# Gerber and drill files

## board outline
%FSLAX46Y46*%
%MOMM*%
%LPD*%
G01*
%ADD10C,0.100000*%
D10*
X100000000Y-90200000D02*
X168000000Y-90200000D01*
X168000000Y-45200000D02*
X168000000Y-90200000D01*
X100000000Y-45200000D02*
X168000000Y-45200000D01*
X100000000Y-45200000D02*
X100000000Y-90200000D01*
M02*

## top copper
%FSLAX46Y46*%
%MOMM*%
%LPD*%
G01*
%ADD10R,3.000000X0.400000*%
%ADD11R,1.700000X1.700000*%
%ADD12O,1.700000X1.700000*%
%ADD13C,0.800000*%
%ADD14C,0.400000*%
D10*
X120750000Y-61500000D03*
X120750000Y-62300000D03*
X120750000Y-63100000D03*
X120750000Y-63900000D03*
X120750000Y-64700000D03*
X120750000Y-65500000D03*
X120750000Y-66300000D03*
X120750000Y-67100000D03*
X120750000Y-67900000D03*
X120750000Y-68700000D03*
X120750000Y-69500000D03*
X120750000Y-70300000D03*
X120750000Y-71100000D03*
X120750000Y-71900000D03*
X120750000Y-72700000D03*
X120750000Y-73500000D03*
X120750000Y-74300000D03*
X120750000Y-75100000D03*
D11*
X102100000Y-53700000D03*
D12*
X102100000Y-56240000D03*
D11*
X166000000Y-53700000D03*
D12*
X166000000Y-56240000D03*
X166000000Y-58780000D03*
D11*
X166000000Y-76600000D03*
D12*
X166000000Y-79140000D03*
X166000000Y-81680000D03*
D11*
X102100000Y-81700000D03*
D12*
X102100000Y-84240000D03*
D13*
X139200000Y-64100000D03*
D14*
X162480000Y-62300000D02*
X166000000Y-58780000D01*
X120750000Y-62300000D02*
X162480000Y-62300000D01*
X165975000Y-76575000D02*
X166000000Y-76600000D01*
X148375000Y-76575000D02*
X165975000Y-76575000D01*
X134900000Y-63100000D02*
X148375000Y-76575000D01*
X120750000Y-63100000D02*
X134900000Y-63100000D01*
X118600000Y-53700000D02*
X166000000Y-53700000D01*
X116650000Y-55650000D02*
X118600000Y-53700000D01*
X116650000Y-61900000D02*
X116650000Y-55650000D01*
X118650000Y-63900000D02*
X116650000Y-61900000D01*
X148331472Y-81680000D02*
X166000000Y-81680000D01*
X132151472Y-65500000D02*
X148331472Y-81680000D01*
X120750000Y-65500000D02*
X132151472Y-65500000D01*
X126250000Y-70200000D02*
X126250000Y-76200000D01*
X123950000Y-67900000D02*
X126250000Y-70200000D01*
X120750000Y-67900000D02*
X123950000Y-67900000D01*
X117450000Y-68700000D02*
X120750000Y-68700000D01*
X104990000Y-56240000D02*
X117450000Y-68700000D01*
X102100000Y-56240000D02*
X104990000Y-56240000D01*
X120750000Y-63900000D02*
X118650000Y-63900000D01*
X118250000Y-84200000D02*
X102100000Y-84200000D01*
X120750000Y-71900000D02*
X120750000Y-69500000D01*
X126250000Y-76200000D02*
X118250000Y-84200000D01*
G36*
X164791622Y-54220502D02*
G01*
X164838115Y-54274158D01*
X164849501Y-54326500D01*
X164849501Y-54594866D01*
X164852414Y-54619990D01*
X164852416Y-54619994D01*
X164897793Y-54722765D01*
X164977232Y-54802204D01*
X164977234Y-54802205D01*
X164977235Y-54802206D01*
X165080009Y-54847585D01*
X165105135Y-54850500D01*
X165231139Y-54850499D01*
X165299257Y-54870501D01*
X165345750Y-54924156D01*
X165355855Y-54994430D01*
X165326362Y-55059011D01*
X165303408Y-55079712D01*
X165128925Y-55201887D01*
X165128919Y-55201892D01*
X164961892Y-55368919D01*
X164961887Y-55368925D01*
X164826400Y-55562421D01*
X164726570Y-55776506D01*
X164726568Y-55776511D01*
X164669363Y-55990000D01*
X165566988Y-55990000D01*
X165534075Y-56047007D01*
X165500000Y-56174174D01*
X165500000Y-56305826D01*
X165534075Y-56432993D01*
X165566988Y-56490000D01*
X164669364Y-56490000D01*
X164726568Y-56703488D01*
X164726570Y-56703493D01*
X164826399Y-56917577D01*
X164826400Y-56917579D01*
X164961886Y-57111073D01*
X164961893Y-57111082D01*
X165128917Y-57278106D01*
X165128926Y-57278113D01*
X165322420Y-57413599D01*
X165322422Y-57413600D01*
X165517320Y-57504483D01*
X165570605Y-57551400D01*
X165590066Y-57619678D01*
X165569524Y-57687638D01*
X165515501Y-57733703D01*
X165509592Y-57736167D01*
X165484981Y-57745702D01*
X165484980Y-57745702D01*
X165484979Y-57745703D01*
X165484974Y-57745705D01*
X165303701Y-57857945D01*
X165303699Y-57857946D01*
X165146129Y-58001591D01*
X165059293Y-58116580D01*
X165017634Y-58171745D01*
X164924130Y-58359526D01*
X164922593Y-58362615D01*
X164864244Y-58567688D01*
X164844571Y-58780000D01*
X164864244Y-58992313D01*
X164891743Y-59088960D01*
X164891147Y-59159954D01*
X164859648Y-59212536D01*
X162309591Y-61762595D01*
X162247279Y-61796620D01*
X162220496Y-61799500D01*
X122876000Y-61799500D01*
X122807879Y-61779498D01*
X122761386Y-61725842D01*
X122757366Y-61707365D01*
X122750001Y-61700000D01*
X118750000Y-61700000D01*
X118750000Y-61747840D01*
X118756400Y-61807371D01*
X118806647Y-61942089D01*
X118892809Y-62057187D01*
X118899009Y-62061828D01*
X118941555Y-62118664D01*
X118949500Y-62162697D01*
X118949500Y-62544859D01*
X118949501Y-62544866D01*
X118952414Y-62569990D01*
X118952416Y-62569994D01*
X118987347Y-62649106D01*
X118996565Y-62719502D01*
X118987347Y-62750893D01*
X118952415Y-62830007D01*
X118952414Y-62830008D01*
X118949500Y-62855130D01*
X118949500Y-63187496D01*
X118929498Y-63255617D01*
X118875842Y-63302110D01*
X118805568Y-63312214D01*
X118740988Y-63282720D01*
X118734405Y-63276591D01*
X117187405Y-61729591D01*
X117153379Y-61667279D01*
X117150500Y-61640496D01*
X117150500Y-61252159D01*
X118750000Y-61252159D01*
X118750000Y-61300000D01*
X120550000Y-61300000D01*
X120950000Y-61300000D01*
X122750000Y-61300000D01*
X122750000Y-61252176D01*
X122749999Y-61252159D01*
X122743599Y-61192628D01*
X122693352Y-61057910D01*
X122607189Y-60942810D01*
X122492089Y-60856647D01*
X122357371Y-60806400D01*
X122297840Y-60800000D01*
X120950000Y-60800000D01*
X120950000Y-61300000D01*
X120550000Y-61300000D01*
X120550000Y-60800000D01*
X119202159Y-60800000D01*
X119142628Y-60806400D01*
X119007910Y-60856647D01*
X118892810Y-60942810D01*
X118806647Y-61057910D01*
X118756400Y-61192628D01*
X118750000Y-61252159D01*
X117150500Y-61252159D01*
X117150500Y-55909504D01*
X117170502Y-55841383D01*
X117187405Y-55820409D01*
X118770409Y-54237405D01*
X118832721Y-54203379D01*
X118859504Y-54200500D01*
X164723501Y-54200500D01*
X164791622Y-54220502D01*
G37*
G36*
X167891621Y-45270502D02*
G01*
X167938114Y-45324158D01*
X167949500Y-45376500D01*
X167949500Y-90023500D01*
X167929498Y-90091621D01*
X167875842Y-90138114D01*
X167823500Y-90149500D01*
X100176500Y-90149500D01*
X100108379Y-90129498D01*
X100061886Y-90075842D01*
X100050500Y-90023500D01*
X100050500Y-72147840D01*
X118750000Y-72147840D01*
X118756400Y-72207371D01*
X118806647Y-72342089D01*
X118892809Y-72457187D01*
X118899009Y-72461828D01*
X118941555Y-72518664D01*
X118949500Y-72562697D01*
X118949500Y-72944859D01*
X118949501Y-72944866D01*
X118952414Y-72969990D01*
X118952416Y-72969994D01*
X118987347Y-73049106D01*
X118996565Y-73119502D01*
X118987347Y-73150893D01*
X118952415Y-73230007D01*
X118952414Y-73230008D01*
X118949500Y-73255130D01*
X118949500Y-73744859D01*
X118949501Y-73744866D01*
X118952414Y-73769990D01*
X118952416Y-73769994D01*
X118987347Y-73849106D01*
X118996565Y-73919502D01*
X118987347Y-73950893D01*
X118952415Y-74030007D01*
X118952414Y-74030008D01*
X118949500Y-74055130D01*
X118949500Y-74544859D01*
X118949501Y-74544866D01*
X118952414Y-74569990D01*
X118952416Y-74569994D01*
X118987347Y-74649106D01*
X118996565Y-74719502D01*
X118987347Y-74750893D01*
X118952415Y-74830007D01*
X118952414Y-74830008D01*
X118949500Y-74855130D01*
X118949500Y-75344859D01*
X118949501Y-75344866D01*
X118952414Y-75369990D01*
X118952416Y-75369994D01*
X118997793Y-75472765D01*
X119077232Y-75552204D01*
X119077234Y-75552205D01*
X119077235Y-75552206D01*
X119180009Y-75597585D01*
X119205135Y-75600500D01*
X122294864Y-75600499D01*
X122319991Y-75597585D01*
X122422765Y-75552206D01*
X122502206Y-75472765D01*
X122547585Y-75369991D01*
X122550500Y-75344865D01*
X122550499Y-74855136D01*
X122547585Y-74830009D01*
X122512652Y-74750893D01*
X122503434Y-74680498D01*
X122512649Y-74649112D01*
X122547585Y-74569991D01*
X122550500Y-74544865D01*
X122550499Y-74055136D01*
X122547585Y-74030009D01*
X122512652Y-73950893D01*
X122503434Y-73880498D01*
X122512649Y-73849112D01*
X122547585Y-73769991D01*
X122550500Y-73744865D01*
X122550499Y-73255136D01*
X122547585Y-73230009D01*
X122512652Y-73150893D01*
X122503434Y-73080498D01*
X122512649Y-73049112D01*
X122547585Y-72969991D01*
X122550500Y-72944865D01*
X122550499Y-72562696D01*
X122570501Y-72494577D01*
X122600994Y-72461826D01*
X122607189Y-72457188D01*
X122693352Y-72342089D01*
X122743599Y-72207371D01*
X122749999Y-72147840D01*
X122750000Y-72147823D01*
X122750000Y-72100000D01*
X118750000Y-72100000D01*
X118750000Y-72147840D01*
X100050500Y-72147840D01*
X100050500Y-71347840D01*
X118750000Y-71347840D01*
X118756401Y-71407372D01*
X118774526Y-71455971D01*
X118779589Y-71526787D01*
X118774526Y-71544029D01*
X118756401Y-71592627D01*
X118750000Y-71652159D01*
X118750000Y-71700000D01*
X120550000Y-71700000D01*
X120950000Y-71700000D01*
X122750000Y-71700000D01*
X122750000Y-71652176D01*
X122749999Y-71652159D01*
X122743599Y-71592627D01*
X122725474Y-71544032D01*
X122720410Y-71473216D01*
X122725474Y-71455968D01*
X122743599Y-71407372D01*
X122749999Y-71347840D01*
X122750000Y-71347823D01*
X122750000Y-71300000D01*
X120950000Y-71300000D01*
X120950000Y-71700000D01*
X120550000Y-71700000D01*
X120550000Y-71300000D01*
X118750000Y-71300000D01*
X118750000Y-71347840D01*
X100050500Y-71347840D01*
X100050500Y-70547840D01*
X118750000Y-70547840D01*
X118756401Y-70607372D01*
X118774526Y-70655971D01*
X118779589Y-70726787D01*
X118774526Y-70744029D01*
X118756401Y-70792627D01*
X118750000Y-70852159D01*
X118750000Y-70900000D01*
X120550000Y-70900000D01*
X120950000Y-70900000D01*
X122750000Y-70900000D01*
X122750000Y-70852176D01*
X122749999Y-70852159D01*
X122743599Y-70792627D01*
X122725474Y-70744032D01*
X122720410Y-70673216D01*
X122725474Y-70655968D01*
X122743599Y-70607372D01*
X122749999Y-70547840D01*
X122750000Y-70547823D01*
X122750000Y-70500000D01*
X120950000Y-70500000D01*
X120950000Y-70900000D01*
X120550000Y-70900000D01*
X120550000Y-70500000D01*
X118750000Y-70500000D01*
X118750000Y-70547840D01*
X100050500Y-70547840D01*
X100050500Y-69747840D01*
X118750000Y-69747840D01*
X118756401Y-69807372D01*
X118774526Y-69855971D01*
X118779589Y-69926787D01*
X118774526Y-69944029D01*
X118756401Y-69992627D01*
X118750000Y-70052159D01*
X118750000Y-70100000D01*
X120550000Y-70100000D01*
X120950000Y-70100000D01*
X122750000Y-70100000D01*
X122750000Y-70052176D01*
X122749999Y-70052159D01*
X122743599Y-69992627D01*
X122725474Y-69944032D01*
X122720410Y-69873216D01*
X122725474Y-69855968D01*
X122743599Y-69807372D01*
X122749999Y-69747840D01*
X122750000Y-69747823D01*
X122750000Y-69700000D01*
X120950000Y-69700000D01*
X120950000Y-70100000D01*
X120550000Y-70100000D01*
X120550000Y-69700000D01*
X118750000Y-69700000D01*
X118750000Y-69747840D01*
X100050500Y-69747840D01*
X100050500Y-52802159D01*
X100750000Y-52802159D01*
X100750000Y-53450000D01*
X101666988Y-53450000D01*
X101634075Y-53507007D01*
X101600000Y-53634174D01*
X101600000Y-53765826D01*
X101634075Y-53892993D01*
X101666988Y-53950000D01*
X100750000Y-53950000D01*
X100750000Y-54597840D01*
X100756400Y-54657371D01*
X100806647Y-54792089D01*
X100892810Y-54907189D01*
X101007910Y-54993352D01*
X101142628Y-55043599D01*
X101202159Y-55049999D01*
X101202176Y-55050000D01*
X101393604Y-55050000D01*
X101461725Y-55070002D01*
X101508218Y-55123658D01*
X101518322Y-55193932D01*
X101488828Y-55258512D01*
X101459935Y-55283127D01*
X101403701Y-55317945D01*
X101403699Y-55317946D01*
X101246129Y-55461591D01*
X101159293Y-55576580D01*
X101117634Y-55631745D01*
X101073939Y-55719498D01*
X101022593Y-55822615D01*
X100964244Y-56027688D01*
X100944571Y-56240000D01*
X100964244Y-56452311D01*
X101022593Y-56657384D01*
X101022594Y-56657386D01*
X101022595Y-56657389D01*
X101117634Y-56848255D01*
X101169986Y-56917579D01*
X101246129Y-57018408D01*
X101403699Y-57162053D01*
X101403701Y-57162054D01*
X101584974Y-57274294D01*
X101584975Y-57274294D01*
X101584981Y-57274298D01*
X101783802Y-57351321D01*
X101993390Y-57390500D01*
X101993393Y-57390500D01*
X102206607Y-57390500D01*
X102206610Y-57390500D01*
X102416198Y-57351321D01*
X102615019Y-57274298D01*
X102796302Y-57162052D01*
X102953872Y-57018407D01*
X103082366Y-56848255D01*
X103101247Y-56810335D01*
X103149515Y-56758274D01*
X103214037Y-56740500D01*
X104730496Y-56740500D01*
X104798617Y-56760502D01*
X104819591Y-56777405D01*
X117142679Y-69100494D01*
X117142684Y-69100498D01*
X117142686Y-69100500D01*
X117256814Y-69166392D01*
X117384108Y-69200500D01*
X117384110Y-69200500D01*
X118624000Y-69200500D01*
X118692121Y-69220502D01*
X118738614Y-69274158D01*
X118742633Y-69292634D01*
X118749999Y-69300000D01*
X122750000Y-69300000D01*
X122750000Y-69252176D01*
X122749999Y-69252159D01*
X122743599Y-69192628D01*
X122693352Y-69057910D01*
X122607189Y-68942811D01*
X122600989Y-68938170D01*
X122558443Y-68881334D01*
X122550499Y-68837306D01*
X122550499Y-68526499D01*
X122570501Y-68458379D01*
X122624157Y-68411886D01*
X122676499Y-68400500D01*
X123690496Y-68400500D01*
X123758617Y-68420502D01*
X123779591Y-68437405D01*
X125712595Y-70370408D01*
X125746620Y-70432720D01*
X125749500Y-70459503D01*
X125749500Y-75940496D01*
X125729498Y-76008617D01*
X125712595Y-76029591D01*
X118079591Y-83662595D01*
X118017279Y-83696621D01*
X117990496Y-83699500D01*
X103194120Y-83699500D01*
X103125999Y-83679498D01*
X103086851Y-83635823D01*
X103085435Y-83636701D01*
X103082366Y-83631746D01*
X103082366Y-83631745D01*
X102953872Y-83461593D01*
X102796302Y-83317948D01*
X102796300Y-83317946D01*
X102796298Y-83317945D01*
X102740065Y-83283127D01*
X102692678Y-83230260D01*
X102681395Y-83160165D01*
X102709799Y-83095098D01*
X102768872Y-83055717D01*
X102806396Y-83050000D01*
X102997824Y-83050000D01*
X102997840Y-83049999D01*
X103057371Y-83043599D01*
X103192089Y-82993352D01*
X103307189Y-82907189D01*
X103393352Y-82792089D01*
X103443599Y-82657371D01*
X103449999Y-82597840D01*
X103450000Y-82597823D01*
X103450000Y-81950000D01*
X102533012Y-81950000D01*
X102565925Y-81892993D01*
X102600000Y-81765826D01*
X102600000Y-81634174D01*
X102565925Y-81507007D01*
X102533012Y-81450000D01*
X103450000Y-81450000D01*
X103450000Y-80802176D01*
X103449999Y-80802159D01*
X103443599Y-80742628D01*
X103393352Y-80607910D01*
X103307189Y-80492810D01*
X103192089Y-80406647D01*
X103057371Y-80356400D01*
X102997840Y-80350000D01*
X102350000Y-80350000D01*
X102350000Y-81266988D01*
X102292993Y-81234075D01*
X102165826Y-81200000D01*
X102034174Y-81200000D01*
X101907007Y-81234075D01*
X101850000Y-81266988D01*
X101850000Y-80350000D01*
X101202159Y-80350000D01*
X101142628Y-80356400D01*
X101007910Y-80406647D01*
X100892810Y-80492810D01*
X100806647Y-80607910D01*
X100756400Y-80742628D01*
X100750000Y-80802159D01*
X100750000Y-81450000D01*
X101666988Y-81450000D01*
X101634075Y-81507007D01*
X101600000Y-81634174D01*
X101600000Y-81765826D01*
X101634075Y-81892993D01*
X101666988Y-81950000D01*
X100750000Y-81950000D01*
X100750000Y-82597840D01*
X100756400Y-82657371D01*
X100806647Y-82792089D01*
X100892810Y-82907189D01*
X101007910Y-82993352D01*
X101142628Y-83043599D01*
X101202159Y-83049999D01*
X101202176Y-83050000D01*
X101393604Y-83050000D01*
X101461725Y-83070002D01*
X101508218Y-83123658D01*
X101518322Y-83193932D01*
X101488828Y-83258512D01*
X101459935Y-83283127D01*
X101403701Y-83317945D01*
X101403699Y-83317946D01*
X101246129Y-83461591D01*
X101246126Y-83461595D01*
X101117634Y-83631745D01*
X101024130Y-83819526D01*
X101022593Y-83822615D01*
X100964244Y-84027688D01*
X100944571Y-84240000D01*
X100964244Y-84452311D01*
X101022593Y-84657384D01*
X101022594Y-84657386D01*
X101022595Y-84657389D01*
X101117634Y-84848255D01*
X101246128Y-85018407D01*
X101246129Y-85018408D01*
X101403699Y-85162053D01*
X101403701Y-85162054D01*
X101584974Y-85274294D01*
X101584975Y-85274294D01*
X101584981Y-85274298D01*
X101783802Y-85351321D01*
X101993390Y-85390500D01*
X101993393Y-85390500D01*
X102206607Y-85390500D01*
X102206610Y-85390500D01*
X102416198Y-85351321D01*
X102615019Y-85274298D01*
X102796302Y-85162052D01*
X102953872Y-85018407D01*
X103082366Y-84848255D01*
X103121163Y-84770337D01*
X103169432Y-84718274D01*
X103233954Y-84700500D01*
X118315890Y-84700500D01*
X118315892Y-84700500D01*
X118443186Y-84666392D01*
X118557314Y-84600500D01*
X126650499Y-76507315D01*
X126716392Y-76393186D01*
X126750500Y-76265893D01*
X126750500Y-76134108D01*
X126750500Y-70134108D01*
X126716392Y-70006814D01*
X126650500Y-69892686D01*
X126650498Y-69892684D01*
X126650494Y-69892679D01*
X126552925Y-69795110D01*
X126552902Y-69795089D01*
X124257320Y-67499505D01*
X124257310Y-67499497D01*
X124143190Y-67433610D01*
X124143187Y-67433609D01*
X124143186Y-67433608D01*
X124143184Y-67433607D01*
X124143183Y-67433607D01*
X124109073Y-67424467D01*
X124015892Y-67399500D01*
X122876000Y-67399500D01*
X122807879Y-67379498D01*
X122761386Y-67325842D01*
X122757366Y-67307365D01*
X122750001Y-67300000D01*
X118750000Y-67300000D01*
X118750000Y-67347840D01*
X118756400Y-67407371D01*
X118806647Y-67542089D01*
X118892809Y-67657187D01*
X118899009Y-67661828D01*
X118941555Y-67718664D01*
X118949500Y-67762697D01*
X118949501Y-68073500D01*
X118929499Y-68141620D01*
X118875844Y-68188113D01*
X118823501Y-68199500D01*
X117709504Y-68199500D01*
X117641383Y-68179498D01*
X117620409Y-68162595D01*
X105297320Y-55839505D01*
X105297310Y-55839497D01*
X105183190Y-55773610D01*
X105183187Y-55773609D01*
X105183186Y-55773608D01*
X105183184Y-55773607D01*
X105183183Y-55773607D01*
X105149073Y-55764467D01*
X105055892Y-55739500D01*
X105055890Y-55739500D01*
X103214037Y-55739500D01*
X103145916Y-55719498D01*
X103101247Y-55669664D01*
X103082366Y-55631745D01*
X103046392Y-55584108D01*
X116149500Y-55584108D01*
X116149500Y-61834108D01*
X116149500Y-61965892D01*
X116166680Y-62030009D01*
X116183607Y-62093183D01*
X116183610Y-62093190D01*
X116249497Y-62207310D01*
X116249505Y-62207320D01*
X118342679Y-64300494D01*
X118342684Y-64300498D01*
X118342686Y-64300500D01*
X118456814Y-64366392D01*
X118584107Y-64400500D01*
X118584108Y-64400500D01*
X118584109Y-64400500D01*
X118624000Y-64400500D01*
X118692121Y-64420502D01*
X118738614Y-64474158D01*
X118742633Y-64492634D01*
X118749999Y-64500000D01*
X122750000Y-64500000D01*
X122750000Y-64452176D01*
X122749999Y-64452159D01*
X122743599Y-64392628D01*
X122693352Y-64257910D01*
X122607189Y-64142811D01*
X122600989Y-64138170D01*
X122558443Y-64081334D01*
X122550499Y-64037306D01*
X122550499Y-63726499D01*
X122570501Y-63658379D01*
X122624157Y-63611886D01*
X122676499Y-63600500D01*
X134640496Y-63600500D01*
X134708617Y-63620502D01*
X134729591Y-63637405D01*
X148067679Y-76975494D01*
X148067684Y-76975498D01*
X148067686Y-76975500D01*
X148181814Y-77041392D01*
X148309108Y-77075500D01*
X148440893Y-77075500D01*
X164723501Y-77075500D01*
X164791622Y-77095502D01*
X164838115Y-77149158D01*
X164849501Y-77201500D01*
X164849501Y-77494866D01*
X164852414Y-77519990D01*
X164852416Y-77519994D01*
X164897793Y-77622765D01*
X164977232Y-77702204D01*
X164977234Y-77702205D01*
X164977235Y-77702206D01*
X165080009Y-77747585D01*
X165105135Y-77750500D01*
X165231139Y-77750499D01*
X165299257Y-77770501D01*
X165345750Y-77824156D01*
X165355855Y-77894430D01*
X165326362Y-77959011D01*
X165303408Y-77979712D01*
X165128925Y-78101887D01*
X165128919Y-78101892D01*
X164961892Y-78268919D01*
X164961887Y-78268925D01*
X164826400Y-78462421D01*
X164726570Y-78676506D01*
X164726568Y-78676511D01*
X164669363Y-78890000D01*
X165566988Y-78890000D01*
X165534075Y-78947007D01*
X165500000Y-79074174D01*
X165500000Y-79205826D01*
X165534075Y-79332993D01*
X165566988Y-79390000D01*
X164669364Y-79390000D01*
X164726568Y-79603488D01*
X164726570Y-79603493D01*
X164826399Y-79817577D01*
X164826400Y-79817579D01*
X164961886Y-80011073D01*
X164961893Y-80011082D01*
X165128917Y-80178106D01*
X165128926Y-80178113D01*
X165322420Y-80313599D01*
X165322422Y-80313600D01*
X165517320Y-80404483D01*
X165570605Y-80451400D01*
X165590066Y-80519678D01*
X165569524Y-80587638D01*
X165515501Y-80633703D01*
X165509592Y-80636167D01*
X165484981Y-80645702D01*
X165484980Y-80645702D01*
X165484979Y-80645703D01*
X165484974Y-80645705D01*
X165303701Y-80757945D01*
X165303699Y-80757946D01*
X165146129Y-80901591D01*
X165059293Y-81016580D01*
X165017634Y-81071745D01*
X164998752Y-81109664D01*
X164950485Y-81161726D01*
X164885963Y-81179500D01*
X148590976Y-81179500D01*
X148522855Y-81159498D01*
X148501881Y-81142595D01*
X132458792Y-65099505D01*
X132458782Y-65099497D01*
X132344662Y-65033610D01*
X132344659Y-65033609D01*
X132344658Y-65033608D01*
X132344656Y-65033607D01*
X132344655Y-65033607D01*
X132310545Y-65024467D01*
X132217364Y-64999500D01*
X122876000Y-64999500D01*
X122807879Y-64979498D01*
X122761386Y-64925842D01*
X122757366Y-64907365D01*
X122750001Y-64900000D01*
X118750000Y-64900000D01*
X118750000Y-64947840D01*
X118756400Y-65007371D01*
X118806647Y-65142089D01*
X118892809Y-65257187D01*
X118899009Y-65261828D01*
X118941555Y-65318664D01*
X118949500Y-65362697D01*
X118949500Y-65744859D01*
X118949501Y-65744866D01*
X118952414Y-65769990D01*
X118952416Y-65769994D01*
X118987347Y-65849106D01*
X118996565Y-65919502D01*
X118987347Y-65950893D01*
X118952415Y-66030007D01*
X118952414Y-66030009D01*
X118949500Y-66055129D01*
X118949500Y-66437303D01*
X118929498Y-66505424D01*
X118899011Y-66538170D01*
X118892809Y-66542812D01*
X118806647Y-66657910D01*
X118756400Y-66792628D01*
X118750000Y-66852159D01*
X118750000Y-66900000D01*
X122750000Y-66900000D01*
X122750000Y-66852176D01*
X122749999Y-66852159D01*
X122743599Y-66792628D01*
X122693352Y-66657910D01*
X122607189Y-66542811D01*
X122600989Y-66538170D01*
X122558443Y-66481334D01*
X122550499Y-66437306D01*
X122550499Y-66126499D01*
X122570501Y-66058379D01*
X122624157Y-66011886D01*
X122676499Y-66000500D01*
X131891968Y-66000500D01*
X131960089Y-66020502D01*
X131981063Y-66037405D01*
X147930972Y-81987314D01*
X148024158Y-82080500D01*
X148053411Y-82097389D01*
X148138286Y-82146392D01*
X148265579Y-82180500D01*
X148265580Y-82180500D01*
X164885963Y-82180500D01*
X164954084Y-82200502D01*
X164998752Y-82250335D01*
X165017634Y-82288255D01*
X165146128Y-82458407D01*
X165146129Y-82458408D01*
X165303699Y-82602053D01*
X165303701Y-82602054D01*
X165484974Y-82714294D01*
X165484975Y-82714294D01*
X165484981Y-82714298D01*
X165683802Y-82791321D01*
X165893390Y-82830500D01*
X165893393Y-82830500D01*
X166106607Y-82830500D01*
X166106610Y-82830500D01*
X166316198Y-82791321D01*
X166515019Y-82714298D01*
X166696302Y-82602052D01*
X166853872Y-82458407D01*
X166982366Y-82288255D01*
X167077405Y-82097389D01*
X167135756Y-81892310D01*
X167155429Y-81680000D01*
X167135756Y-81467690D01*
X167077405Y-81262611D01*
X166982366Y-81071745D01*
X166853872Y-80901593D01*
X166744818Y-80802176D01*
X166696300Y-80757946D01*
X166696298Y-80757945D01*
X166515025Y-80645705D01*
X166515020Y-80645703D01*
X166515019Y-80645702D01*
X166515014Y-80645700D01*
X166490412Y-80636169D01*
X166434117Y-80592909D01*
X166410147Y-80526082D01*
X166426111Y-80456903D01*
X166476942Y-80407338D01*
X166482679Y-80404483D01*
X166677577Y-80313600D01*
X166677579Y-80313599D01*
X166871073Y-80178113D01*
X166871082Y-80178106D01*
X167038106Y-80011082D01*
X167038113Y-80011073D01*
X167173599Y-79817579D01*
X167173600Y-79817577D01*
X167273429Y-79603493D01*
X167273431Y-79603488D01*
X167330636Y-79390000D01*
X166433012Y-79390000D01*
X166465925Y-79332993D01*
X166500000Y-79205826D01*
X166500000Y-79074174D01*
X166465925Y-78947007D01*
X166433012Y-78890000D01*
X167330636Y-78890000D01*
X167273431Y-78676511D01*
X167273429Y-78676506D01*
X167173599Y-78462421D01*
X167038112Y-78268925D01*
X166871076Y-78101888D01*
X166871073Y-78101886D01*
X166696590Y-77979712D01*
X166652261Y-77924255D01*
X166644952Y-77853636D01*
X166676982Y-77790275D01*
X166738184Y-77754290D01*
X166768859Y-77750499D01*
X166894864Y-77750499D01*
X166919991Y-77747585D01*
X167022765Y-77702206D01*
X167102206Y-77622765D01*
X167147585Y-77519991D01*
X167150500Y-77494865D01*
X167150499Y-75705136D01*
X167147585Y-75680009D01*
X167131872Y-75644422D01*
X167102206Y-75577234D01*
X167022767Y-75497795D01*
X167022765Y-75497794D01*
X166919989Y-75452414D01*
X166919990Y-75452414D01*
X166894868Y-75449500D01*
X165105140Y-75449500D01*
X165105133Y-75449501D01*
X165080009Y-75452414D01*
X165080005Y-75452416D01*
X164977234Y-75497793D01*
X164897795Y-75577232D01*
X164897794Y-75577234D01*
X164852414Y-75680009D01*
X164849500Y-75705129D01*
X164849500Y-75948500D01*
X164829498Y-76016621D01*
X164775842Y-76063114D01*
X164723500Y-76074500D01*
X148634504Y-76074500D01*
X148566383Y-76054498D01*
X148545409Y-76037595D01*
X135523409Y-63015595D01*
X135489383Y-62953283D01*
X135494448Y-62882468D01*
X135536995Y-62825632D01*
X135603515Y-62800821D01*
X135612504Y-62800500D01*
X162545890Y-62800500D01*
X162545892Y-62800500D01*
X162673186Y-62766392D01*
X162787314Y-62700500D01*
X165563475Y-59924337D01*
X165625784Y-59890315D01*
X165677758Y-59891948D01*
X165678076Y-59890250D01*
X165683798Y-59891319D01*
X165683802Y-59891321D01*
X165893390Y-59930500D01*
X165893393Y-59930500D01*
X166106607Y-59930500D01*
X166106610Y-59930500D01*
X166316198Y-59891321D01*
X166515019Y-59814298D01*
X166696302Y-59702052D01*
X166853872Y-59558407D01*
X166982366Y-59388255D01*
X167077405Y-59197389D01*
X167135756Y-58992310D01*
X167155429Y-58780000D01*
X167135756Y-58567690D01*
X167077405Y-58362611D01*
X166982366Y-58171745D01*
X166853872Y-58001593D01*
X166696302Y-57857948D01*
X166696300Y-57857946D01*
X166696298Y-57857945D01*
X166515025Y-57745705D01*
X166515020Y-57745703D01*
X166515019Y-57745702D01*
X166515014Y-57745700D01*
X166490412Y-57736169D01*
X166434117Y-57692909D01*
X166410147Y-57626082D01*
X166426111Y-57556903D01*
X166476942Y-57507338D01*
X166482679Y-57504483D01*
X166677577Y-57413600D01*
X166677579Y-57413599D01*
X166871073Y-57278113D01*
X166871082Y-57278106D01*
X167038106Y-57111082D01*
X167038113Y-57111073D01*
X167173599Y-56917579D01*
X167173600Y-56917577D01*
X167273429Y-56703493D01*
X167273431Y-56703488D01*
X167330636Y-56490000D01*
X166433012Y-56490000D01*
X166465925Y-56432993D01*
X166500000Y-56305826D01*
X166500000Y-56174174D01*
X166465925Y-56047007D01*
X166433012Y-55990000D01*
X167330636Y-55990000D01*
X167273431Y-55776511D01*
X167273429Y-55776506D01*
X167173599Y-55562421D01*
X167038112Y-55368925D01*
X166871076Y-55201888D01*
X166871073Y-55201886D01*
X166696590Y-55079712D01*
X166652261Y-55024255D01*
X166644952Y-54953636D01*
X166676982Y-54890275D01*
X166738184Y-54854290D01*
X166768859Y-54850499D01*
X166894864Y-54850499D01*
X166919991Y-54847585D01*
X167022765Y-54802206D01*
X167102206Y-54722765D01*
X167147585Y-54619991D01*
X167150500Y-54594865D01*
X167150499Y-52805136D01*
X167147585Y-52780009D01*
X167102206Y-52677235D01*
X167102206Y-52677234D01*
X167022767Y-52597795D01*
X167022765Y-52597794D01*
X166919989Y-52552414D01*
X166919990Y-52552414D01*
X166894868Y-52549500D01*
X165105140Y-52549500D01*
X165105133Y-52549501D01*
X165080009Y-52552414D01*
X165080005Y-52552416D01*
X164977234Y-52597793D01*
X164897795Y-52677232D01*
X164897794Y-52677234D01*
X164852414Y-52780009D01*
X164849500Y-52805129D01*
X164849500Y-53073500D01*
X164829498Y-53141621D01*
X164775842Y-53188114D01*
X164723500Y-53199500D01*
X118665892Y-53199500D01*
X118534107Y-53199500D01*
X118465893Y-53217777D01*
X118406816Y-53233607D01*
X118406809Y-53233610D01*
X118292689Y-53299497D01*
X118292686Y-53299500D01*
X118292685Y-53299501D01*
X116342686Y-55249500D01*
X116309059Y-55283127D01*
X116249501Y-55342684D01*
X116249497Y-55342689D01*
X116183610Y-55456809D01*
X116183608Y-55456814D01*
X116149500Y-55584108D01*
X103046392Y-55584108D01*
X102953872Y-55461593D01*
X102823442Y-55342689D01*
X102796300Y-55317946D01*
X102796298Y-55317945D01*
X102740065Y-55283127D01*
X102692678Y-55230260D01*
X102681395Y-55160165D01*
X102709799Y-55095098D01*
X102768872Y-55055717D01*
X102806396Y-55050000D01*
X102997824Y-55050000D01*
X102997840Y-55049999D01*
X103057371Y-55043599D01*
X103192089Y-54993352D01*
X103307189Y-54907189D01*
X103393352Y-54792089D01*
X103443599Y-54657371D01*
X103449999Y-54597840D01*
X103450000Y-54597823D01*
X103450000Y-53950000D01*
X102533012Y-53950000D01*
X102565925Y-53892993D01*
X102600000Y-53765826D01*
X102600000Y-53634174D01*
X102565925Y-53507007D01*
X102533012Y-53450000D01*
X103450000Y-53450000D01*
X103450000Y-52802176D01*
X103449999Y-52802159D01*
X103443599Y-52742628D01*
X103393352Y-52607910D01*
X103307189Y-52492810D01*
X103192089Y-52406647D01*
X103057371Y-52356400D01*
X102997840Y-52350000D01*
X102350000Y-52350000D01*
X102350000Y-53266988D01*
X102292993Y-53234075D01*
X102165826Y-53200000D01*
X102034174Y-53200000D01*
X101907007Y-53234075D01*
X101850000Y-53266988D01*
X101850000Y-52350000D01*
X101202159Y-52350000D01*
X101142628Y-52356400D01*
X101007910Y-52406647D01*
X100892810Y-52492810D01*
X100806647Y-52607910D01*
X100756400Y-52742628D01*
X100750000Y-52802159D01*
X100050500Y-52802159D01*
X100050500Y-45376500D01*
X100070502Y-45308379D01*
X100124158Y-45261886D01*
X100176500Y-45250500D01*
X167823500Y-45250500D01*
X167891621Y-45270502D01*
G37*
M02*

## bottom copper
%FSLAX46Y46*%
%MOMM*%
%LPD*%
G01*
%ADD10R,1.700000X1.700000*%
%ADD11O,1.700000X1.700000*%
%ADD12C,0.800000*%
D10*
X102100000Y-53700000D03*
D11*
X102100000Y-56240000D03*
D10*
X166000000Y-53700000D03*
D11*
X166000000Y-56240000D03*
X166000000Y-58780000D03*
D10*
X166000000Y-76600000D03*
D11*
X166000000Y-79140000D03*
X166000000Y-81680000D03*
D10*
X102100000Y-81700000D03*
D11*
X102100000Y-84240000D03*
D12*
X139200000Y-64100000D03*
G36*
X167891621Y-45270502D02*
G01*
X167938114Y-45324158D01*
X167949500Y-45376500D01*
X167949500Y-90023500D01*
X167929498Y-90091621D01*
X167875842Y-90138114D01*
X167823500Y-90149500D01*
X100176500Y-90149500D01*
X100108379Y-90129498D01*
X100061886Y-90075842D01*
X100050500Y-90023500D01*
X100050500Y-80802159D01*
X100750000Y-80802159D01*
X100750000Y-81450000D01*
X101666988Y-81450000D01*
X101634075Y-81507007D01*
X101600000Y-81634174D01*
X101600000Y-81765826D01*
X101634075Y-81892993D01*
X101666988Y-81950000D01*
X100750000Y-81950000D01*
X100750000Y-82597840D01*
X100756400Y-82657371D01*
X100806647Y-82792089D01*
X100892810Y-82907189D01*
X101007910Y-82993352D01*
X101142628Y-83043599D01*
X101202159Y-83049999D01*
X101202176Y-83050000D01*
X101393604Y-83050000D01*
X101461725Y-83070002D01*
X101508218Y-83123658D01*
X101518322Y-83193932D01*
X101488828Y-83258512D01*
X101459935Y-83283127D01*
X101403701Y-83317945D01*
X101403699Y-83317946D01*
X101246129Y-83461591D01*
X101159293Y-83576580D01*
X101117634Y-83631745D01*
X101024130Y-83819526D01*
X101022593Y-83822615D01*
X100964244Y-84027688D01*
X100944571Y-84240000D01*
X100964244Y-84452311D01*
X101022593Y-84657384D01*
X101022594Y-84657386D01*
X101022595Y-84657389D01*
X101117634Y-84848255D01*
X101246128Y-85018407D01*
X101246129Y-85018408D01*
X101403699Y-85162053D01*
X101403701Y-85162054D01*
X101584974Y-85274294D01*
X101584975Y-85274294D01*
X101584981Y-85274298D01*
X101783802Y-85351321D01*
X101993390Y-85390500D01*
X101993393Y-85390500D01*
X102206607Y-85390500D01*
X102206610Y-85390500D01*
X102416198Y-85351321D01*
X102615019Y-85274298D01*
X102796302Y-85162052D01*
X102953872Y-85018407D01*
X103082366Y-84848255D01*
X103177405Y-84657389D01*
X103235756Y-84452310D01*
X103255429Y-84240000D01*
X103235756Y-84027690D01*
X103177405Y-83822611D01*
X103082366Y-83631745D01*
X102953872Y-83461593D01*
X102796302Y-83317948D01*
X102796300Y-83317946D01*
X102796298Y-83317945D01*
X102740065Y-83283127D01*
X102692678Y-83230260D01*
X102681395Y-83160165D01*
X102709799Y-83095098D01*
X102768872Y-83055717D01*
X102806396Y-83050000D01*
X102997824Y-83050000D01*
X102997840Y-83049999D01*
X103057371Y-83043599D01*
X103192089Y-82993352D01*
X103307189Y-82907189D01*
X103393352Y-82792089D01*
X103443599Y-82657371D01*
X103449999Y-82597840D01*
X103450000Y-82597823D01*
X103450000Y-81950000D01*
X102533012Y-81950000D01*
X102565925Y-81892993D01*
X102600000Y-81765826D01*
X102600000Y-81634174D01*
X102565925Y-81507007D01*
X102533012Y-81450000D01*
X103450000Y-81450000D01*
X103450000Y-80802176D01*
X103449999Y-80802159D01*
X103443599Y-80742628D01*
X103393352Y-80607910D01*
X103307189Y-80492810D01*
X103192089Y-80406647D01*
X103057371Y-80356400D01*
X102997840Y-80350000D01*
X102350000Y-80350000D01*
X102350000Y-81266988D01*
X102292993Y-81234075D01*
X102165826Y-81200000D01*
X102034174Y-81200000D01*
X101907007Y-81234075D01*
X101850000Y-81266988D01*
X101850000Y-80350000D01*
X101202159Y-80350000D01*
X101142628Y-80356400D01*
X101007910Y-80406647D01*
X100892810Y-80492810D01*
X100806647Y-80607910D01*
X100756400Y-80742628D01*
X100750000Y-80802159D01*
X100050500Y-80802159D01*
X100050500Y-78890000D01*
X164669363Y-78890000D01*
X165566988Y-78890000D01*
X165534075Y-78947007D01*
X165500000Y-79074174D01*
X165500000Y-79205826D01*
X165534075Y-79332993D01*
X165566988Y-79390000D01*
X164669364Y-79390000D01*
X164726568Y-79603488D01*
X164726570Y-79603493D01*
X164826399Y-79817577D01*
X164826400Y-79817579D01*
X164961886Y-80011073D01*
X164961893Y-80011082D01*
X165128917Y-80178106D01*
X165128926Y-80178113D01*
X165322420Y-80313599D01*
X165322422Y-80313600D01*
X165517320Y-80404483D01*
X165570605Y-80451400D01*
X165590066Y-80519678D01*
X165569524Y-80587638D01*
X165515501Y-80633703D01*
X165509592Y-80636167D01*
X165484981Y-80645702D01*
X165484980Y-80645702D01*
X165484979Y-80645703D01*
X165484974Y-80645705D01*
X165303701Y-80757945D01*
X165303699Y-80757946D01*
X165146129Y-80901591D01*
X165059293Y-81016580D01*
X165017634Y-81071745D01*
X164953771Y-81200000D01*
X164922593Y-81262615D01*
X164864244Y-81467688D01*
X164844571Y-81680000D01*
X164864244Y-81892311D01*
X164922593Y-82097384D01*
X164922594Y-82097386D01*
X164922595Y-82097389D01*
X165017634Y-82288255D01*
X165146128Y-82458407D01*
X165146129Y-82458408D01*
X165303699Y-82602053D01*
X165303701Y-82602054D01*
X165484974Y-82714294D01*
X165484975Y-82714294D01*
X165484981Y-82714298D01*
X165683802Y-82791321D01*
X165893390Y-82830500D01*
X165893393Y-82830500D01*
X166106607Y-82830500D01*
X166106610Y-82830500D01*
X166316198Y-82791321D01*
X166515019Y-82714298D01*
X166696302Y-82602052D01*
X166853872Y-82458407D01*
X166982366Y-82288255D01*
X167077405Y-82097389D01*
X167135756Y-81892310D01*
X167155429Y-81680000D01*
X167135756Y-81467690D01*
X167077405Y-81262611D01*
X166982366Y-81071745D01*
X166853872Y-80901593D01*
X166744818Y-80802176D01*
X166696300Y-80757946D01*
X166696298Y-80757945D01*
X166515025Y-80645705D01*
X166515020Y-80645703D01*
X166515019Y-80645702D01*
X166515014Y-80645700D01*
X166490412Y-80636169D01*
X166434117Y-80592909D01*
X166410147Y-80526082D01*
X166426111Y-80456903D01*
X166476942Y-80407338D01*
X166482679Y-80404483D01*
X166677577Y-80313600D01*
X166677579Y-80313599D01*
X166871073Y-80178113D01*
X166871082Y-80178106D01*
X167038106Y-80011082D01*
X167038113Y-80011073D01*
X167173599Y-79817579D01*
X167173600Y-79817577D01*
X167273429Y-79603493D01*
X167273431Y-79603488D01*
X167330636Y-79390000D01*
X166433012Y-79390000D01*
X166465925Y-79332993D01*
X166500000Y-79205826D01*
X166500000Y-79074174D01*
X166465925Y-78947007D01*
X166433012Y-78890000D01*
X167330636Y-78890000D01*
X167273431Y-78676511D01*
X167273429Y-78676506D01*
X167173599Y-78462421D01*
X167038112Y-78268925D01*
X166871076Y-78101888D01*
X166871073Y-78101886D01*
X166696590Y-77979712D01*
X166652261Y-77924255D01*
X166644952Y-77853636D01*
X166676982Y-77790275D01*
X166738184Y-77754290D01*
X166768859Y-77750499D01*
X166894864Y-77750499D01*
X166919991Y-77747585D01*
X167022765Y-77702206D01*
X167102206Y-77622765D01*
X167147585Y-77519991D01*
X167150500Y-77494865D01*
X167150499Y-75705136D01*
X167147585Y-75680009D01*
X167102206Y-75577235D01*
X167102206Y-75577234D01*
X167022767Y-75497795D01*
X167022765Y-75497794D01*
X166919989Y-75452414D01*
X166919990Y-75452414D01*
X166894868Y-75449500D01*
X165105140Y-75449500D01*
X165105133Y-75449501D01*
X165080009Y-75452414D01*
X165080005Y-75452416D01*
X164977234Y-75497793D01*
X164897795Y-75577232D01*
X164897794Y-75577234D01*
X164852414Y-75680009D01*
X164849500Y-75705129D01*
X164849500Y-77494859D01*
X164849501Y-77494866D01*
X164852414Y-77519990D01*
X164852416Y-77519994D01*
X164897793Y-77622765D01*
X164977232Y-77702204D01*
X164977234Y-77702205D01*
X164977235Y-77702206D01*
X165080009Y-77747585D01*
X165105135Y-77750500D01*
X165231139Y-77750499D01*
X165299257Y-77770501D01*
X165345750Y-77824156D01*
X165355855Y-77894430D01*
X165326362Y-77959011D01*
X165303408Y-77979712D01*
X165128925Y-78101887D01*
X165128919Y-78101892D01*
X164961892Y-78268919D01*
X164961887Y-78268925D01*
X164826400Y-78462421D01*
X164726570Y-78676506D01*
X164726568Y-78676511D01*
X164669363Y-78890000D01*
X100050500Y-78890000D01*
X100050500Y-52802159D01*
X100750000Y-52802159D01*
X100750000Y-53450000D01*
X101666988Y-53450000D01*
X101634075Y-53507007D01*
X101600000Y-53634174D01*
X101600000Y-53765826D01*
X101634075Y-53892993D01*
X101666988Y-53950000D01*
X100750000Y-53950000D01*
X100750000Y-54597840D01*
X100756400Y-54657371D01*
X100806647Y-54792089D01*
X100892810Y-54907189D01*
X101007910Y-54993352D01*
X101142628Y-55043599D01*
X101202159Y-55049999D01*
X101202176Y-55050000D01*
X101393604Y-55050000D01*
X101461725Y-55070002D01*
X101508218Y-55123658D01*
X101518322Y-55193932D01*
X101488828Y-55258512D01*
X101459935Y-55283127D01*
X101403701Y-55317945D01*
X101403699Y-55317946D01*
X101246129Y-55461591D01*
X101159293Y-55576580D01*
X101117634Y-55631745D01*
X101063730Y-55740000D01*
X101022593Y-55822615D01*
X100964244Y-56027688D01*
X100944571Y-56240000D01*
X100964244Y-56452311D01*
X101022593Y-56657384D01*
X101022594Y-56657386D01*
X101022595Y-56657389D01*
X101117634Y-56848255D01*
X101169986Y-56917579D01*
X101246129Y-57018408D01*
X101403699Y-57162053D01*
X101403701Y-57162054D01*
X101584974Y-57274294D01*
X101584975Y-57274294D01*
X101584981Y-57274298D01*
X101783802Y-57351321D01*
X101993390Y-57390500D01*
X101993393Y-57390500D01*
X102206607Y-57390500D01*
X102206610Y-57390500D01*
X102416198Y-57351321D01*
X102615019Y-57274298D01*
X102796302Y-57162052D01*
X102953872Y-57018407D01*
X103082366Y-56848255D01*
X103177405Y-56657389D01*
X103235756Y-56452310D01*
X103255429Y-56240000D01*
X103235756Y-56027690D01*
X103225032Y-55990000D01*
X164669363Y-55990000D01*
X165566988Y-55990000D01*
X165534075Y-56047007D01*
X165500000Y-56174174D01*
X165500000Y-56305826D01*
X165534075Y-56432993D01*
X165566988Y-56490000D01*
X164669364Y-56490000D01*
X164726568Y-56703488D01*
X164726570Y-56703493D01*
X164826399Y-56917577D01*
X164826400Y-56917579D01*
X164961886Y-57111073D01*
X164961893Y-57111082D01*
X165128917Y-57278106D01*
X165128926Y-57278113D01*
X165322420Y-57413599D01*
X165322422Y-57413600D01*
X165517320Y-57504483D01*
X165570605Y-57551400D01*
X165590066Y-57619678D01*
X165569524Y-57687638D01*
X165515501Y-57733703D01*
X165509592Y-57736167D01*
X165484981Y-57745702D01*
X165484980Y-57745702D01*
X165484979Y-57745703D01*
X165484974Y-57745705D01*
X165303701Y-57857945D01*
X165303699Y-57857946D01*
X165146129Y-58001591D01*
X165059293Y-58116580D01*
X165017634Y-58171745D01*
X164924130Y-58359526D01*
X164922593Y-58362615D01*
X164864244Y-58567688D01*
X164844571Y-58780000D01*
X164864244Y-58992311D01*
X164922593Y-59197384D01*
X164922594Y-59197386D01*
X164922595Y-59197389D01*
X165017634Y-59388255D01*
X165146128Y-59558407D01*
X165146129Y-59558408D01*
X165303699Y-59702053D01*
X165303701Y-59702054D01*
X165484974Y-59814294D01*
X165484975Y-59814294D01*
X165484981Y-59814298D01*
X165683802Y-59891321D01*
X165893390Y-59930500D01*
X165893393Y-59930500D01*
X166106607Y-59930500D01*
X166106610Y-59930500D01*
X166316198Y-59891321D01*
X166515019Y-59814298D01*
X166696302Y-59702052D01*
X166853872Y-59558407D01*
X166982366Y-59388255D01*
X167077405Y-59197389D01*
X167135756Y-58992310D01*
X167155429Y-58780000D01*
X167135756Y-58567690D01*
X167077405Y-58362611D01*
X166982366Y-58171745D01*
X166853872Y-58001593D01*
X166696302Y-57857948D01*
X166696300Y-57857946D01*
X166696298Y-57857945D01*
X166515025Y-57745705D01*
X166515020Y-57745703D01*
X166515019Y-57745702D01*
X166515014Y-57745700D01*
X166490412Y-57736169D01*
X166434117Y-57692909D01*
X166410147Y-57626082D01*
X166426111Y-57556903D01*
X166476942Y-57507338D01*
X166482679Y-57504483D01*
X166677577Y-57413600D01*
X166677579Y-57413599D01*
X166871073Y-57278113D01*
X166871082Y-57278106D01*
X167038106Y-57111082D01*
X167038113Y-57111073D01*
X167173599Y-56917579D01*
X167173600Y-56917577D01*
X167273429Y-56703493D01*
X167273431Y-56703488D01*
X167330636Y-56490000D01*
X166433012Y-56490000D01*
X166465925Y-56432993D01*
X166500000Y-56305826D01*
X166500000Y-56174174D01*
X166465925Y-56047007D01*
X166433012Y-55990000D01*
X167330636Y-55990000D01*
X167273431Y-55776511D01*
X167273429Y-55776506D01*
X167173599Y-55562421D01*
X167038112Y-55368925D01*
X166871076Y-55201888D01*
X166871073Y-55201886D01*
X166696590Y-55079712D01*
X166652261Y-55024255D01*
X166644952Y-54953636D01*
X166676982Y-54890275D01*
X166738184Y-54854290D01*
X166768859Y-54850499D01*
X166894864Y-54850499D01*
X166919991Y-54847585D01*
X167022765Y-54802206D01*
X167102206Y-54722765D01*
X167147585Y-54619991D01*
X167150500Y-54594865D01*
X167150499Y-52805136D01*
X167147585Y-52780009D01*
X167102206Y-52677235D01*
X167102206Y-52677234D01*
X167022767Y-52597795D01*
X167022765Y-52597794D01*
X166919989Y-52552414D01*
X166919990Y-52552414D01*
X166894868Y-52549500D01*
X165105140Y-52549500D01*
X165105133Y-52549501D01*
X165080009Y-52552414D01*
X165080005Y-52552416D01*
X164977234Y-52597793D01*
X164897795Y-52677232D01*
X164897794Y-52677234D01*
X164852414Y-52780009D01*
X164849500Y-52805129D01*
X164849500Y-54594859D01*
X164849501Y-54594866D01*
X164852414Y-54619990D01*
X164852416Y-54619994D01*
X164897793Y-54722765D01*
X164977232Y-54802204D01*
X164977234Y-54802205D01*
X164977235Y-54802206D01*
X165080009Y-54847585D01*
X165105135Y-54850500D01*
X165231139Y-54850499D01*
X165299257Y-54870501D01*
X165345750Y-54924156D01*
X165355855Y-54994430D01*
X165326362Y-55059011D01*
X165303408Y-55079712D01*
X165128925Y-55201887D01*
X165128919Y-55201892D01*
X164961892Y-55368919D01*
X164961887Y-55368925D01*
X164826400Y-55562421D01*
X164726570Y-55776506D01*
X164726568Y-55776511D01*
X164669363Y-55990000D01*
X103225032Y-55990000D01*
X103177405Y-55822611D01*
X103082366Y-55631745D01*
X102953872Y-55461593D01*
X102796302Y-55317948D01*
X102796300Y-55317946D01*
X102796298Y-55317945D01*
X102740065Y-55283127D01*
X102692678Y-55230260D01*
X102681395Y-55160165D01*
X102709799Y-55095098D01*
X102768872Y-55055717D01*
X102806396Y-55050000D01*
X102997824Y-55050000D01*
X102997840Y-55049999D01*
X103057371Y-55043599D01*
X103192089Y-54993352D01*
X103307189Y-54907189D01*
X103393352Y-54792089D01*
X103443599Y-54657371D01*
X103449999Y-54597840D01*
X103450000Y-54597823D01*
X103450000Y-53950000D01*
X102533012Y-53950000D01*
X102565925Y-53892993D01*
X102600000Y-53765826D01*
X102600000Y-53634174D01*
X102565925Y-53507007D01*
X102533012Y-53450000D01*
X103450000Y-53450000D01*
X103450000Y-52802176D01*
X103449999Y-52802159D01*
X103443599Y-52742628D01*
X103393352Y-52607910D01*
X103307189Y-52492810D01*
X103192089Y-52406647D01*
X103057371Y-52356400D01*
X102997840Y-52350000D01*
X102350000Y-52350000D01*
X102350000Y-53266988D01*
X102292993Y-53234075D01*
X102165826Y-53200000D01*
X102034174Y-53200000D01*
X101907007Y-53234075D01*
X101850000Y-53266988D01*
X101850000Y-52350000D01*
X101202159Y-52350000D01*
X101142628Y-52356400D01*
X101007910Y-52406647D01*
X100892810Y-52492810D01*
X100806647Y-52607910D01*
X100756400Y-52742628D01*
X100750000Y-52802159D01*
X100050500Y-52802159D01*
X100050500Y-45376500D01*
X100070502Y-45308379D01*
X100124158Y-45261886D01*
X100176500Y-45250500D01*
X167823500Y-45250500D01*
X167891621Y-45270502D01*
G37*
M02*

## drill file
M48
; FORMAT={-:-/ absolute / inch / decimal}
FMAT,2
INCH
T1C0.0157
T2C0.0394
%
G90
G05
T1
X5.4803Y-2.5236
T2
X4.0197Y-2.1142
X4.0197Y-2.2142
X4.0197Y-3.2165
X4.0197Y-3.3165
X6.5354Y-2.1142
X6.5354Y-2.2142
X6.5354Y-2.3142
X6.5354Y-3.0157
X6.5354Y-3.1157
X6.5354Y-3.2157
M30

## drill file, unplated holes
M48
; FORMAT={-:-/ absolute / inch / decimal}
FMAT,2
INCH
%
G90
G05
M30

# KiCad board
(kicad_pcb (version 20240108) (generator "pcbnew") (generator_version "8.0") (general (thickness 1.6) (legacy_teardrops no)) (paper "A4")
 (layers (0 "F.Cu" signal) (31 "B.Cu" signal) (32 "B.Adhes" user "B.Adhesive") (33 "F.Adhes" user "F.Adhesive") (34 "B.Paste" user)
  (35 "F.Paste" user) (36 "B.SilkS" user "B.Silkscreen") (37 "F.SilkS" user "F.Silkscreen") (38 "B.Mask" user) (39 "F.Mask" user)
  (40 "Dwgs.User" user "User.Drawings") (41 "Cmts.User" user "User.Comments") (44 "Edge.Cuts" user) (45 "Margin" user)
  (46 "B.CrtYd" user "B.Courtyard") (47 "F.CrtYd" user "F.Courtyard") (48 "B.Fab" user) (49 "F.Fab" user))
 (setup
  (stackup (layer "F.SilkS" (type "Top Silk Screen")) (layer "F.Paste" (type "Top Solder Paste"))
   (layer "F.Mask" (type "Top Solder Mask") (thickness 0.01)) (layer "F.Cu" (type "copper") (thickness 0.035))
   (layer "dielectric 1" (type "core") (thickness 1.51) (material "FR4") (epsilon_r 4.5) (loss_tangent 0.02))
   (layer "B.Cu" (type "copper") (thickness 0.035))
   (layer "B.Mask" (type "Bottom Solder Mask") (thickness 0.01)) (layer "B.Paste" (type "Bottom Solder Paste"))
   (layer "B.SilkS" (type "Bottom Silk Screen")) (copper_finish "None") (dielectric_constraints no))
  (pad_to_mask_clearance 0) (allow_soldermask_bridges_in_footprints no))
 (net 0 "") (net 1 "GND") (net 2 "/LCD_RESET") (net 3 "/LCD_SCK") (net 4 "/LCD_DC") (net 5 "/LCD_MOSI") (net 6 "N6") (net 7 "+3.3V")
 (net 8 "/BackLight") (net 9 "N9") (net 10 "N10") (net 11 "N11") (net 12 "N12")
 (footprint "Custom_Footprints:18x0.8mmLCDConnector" (layer "F.Cu") (at 120.75 61.5 -90)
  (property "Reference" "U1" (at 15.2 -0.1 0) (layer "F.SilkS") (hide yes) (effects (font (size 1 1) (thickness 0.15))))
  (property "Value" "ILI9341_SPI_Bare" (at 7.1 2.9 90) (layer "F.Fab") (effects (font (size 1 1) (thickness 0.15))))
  (pad "1" smd rect (at 0 0 270) (size 0.4 3) (layers "F.Cu" "F.Paste" "F.Mask") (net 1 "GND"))
  (pad "2" smd rect (at 0.8 0 270) (size 0.4 3) (layers "F.Cu" "F.Paste" "F.Mask") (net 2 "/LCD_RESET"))
  (pad "3" smd rect (at 1.6 0 270) (size 0.4 3) (layers "F.Cu" "F.Paste" "F.Mask") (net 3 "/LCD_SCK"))
  (pad "4" smd rect (at 2.4 0 270) (size 0.4 3) (layers "F.Cu" "F.Paste" "F.Mask") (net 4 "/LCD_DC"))
  (pad "5" smd rect (at 3.2 0 270) (size 0.4 3) (layers "F.Cu" "F.Paste" "F.Mask") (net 1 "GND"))
  (pad "6" smd rect (at 4 0 270) (size 0.4 3) (layers "F.Cu" "F.Paste" "F.Mask") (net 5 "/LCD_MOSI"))
  (pad "7" smd rect (at 4.8 0 270) (size 0.4 3) (layers "F.Cu" "F.Paste" "F.Mask") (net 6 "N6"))
  (pad "8" smd rect (at 5.6 0 270) (size 0.4 3) (layers "F.Cu" "F.Paste" "F.Mask") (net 1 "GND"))
  (pad "9" smd rect (at 6.4 0 270) (size 0.4 3) (layers "F.Cu" "F.Paste" "F.Mask") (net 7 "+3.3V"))
  (pad "10" smd rect (at 7.2 0 270) (size 0.4 3) (layers "F.Cu" "F.Paste" "F.Mask") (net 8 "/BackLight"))
  (pad "11" smd rect (at 8 0 270) (size 0.4 3) (layers "F.Cu" "F.Paste" "F.Mask") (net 1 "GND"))
  (pad "12" smd rect (at 8.8 0 270) (size 0.4 3) (layers "F.Cu" "F.Paste" "F.Mask") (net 1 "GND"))
  (pad "13" smd rect (at 9.6 0 270) (size 0.4 3) (layers "F.Cu" "F.Paste" "F.Mask") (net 1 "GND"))
  (pad "14" smd rect (at 10.4 0 270) (size 0.4 3) (layers "F.Cu" "F.Paste" "F.Mask") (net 1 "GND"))
  (pad "15" smd rect (at 11.2 0 270) (size 0.4 3) (layers "F.Cu" "F.Paste" "F.Mask") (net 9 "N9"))
  (pad "16" smd rect (at 12 0 270) (size 0.4 3) (layers "F.Cu" "F.Paste" "F.Mask") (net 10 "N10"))
  (pad "17" smd rect (at 12.8 0 270) (size 0.4 3) (layers "F.Cu" "F.Paste" "F.Mask") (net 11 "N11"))
  (pad "18" smd rect (at 13.6 0 270) (size 0.4 3) (layers "F.Cu" "F.Paste" "F.Mask") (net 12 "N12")))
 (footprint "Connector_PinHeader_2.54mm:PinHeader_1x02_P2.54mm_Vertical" (layer "B.Cu") (at 102.1 53.7 180)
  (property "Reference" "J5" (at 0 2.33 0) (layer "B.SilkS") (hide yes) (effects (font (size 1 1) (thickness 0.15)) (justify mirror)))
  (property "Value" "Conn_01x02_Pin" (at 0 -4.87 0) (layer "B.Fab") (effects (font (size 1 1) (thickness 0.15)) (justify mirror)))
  (pad "1" thru_hole rect (at 0 0 180) (size 1.7 1.7) (drill 1) (layers "*.Cu" "*.Mask") (remove_unused_layers no) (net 1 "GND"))
  (pad "2" thru_hole oval (at 0 -2.54 180) (size 1.7 1.7) (drill 1) (layers "*.Cu" "*.Mask") (remove_unused_layers no) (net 8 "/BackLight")))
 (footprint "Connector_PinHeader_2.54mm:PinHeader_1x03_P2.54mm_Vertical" (layer "B.Cu") (at 166 53.7 180)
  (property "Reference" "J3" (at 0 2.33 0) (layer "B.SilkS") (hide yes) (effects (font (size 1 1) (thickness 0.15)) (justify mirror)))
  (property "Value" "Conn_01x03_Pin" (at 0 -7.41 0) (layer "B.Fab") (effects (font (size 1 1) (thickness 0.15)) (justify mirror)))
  (pad "1" thru_hole rect (at 0 0 180) (size 1.7 1.7) (drill 1) (layers "*.Cu" "*.Mask") (remove_unused_layers no) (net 4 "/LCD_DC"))
  (pad "2" thru_hole oval (at 0 -2.54 180) (size 1.7 1.7) (drill 1) (layers "*.Cu" "*.Mask") (remove_unused_layers no) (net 1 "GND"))
  (pad "3" thru_hole oval (at 0 -5.08 180) (size 1.7 1.7) (drill 1) (layers "*.Cu" "*.Mask") (remove_unused_layers no) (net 2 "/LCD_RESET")))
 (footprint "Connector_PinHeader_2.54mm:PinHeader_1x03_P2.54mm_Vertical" (layer "B.Cu") (at 166 76.6 180)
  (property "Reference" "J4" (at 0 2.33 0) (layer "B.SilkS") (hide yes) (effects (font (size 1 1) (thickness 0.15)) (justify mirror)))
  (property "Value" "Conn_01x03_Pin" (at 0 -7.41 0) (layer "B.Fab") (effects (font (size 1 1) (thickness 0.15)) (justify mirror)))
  (pad "1" thru_hole rect (at 0 0 180) (size 1.7 1.7) (drill 1) (layers "*.Cu" "*.Mask") (remove_unused_layers no) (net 3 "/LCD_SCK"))
  (pad "2" thru_hole oval (at 0 -2.54 180) (size 1.7 1.7) (drill 1) (layers "*.Cu" "*.Mask") (remove_unused_layers no) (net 1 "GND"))
  (pad "3" thru_hole oval (at 0 -5.08 180) (size 1.7 1.7) (drill 1) (layers "*.Cu" "*.Mask") (remove_unused_layers no) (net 5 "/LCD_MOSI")))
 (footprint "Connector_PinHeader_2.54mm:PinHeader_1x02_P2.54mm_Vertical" (layer "B.Cu") (at 102.1 81.7 180)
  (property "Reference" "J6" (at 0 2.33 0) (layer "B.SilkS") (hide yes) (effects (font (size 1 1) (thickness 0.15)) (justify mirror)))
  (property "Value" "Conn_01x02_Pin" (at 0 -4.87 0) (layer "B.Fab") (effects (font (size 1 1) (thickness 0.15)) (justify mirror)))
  (pad "1" thru_hole rect (at 0 0 180) (size 1.7 1.7) (drill 1) (layers "*.Cu" "*.Mask") (remove_unused_layers no) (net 1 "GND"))
  (pad "2" thru_hole oval (at 0 -2.54 180) (size 1.7 1.7) (drill 1) (layers "*.Cu" "*.Mask") (remove_unused_layers no) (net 7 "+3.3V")))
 (gr_line (start 100 90.2) (end 168 90.2) (stroke (width 0.1) (type solid)) (layer "Edge.Cuts"))
 (gr_line (start 168 45.2) (end 168 90.2) (stroke (width 0.1) (type solid)) (layer "Edge.Cuts"))
 (gr_line (start 100 45.2) (end 168 45.2) (stroke (width 0.1) (type solid)) (layer "Edge.Cuts"))
 (gr_line (start 100 45.2) (end 100 90.2) (stroke (width 0.1) (type solid)) (layer "Edge.Cuts"))
 (segment (start 120.75 71.9) (end 120.75 69.5) (width 0.4) (layer "F.Cu") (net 1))
 (via (at 139.2 64.1) (size 0.8) (drill 0.4) (layers "F.Cu" "B.Cu") (free yes) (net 1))
 (segment (start 120.75 67.9) (end 123.95 67.9) (width 0.4) (layer "F.Cu") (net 7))
 (segment (start 118.25 84.2) (end 102.1 84.2) (width 0.4) (layer "F.Cu") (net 7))
 (segment (start 123.95 67.9) (end 126.25 70.2) (width 0.4) (layer "F.Cu") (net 7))
 (segment (start 126.25 70.2) (end 126.25 76.2) (width 0.4) (layer "F.Cu") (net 7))
 (segment (start 126.25 76.2) (end 118.25 84.2) (width 0.4) (layer "F.Cu") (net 7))
 (segment (start 118.65 63.9) (end 116.65 61.9) (width 0.4) (layer "F.Cu") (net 4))
 (segment (start 116.65 61.9) (end 116.65 55.65) (width 0.4) (layer "F.Cu") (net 4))
 (segment (start 120.75 63.9) (end 118.65 63.9) (width 0.4) (layer "F.Cu") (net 4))
 (segment (start 116.65 55.65) (end 118.6 53.7) (width 0.4) (layer "F.Cu") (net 4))
 (segment (start 118.6 53.7) (end 166 53.7) (width 0.4) (layer "F.Cu") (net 4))
 (segment (start 162.48 62.3) (end 166 58.78) (width 0.4) (layer "F.Cu") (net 2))
 (segment (start 120.75 62.3) (end 162.48 62.3) (width 0.4) (layer "F.Cu") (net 2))
 (segment (start 120.75 65.5) (end 132.151472 65.5) (width 0.4) (layer "F.Cu") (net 5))
 (segment (start 132.151472 65.5) (end 148.331472 81.68) (width 0.4) (layer "F.Cu") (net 5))
 (segment (start 148.331472 81.68) (end 166 81.68) (width 0.4) (layer "F.Cu") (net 5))
 (segment (start 102.1 56.24) (end 104.99 56.24) (width 0.4) (layer "F.Cu") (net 8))
 (segment (start 117.45 68.7) (end 120.75 68.7) (width 0.4) (layer "F.Cu") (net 8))
 (segment (start 104.99 56.24) (end 117.45 68.7) (width 0.4) (layer "F.Cu") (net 8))
 (segment (start 134.9 63.1) (end 148.375 76.575) (width 0.4) (layer "F.Cu") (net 3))
 (segment (start 120.75 63.1) (end 134.9 63.1) (width 0.4) (layer "F.Cu") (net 3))
 (segment (start 165.975 76.575) (end 166 76.6) (width 0.4) (layer "F.Cu") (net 3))
 (segment (start 148.375 76.575) (end 165.975 76.575) (width 0.4) (layer "F.Cu") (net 3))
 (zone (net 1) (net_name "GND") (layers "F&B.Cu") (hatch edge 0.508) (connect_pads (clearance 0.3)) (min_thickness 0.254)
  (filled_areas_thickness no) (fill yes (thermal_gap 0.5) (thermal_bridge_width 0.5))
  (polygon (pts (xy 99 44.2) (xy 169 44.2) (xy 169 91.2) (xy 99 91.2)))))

